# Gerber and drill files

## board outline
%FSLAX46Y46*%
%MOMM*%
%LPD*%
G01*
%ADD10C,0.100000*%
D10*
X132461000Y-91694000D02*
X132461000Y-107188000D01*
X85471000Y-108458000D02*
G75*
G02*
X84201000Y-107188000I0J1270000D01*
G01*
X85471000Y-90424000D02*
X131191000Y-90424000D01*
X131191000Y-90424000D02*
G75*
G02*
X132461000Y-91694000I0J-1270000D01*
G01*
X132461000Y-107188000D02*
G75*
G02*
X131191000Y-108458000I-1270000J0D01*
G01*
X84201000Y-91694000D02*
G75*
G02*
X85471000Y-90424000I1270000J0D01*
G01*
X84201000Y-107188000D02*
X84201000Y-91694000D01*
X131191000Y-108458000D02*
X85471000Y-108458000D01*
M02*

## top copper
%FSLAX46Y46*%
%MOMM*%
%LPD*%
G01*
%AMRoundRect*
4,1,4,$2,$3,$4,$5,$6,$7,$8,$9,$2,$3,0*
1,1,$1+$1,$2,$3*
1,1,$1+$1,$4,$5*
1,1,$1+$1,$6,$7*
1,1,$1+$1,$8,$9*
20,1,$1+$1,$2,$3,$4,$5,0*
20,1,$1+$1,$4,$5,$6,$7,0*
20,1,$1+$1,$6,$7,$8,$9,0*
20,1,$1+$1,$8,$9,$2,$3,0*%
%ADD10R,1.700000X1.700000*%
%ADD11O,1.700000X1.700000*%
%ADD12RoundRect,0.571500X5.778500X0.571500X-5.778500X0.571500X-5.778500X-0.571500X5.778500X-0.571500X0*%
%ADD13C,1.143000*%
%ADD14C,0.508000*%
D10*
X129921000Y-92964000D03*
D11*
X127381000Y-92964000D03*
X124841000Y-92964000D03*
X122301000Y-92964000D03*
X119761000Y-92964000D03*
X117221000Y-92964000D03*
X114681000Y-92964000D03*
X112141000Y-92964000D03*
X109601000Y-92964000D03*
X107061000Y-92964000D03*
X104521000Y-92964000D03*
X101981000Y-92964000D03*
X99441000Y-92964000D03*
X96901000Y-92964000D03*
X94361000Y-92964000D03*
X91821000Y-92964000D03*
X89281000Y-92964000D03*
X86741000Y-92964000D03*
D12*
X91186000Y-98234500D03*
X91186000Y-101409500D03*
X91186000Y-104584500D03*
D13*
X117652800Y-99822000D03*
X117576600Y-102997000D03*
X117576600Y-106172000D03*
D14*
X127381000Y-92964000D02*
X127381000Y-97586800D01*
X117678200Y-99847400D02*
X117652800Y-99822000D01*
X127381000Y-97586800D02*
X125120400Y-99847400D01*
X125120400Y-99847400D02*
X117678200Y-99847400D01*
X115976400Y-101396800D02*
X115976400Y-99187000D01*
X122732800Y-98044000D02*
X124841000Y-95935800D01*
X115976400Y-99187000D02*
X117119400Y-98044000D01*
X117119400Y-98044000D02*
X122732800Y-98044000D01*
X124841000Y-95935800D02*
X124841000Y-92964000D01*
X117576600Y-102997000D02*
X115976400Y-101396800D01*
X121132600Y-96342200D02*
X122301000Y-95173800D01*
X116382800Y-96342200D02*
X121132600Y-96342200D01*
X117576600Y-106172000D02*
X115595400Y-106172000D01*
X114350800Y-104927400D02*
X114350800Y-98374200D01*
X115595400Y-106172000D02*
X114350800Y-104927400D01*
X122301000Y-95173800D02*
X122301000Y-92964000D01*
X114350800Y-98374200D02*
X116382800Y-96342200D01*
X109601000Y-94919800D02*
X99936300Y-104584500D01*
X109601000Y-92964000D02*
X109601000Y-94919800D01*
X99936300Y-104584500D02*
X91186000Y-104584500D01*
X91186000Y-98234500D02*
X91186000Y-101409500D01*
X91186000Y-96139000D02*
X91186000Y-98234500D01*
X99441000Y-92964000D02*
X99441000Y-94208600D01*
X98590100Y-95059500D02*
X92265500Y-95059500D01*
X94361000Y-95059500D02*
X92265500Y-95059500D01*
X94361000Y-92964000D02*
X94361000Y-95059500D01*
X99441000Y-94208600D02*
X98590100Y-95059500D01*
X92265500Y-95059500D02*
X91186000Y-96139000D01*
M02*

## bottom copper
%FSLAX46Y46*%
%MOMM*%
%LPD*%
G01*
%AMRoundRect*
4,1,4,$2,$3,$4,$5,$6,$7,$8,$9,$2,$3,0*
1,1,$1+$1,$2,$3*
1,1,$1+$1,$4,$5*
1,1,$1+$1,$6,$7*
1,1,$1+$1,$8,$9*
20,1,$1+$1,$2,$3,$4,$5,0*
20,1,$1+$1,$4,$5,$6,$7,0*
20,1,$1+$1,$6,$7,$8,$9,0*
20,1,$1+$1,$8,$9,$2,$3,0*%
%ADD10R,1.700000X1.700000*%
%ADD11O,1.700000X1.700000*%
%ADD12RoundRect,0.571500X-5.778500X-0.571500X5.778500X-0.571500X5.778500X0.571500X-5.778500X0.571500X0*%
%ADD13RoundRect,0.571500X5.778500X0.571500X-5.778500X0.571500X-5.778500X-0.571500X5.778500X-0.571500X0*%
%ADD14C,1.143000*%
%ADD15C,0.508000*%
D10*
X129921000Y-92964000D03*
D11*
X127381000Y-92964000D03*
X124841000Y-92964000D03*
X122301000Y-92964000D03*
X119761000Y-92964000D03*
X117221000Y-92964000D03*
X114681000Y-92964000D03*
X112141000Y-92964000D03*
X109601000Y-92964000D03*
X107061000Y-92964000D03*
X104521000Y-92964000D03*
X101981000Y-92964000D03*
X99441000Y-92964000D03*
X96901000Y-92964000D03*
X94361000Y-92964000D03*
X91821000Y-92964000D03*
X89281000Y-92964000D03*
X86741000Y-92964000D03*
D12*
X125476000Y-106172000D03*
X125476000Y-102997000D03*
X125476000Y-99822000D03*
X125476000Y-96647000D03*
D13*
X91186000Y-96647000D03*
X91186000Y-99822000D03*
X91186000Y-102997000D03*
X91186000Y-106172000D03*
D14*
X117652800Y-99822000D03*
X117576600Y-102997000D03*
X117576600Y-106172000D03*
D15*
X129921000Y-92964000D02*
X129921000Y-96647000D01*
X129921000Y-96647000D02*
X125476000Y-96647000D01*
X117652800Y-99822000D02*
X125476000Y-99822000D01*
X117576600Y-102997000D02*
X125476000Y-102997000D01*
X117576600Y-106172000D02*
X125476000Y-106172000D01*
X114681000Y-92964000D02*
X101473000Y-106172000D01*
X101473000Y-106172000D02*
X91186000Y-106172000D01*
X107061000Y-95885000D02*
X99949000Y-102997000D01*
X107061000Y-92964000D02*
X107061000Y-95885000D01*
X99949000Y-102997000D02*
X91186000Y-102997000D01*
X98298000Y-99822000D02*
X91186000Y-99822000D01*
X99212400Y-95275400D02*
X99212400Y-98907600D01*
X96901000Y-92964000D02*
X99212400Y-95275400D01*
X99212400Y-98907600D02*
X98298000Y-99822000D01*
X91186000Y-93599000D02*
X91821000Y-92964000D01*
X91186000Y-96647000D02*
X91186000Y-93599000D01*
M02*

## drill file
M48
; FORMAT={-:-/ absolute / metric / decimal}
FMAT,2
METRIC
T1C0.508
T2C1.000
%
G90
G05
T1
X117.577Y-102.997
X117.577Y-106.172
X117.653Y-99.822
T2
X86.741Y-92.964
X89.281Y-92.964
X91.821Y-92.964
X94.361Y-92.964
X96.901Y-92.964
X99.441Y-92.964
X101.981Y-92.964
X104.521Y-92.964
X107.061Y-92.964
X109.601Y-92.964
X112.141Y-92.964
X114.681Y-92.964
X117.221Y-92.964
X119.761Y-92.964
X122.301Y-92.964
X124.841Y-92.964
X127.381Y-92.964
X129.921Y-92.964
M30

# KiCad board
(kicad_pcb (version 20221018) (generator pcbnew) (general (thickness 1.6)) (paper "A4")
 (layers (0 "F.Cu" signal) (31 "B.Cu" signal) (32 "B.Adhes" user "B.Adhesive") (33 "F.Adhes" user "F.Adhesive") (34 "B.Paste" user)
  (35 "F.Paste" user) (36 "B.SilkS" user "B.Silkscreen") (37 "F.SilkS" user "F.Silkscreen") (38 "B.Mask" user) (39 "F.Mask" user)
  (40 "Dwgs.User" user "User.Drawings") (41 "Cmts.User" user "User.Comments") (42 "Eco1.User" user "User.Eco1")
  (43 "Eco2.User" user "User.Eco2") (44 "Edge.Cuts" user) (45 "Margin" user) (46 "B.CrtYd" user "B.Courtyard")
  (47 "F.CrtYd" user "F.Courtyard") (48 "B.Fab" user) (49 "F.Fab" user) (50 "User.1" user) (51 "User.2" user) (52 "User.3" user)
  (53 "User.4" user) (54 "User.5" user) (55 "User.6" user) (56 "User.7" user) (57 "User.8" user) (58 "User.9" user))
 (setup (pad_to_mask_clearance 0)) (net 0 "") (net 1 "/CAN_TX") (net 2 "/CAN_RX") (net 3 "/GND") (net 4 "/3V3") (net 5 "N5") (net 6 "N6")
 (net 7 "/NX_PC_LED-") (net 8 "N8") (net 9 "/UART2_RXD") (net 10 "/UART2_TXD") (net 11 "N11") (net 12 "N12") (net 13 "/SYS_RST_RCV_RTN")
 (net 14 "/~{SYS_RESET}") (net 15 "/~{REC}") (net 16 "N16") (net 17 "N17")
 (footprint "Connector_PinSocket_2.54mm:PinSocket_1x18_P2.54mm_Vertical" (layer "F.Cu") (at 129.921 92.964 -90)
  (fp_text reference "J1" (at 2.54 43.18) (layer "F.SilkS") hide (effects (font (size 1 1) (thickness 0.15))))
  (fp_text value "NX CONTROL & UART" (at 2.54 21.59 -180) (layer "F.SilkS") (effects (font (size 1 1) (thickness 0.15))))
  (pad "1" thru_hole rect (at 0 0 270) (size 1.7 1.7) (drill 1) (layers "*.Cu" "*.Mask") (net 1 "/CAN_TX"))
  (pad "2" thru_hole oval (at 0 2.54 270) (size 1.7 1.7) (drill 1) (layers "*.Cu" "*.Mask") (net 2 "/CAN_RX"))
  (pad "3" thru_hole oval (at 0 5.08 270) (size 1.7 1.7) (drill 1) (layers "*.Cu" "*.Mask") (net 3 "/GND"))
  (pad "4" thru_hole oval (at 0 7.62 270) (size 1.7 1.7) (drill 1) (layers "*.Cu" "*.Mask") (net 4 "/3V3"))
  (pad "5" thru_hole oval (at 0 10.16 270) (size 1.7 1.7) (drill 1) (layers "*.Cu" "*.Mask") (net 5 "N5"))
  (pad "6" thru_hole oval (at 0 12.7 270) (size 1.7 1.7) (drill 1) (layers "*.Cu" "*.Mask") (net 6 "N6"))
  (pad "7" thru_hole oval (at 0 15.24 270) (size 1.7 1.7) (drill 1) (layers "*.Cu" "*.Mask") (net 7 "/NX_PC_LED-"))
  (pad "8" thru_hole oval (at 0 17.78 270) (size 1.7 1.7) (drill 1) (layers "*.Cu" "*.Mask") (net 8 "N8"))
  (pad "9" thru_hole oval (at 0 20.32 270) (size 1.7 1.7) (drill 1) (layers "*.Cu" "*.Mask") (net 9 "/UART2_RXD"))
  (pad "10" thru_hole oval (at 0 22.86 270) (size 1.7 1.7) (drill 1) (layers "*.Cu" "*.Mask") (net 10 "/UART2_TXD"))
  (pad "11" thru_hole oval (at 0 25.4 270) (size 1.7 1.7) (drill 1) (layers "*.Cu" "*.Mask") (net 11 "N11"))
  (pad "12" thru_hole oval (at 0 27.94 270) (size 1.7 1.7) (drill 1) (layers "*.Cu" "*.Mask") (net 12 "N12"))
  (pad "13" thru_hole oval (at 0 30.48 270) (size 1.7 1.7) (drill 1) (layers "*.Cu" "*.Mask") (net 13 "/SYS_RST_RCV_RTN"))
  (pad "14" thru_hole oval (at 0 33.02 270) (size 1.7 1.7) (drill 1) (layers "*.Cu" "*.Mask") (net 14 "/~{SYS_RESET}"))
  (pad "15" thru_hole oval (at 0 35.56 270) (size 1.7 1.7) (drill 1) (layers "*.Cu" "*.Mask") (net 13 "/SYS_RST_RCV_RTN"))
  (pad "16" thru_hole oval (at 0 38.1 270) (size 1.7 1.7) (drill 1) (layers "*.Cu" "*.Mask") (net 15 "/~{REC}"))
  (pad "17" thru_hole oval (at 0 40.64 270) (size 1.7 1.7) (drill 1) (layers "*.Cu" "*.Mask") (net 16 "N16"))
  (pad "18" thru_hole oval (at 0 43.18 270) (size 1.7 1.7) (drill 1) (layers "*.Cu" "*.Mask") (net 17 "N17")))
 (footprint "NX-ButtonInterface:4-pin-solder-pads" (layer "B.Cu") (at 125.476 106.172)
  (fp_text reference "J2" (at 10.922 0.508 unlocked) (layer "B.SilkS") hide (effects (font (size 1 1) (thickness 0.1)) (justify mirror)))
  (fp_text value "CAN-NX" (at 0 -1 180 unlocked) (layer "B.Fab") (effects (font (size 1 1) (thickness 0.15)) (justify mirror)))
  (pad "1" smd roundrect (at 0 0) (size 12.7 2.286) (layers "B.Cu" "B.Paste" "B.Mask") (roundrect_rratio 0.25) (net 4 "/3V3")
   (thermal_bridge_angle 45))
  (pad "2" smd roundrect (at 0 -3.175) (size 12.7 2.286) (layers "B.Cu" "B.Paste" "B.Mask") (roundrect_rratio 0.25) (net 3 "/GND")
   (thermal_bridge_angle 45))
  (pad "3" smd roundrect (at 0 -6.35) (size 12.7 2.286) (layers "B.Cu" "B.Paste" "B.Mask") (roundrect_rratio 0.25) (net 2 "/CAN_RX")
   (thermal_bridge_angle 45))
  (pad "4" smd roundrect (at 0 -9.525) (size 12.7 2.286) (layers "B.Cu" "B.Paste" "B.Mask") (roundrect_rratio 0.25) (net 1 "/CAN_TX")
   (thermal_bridge_angle 45)))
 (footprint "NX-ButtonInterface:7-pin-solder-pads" (layer "B.Cu") (at 91.186 96.647 180)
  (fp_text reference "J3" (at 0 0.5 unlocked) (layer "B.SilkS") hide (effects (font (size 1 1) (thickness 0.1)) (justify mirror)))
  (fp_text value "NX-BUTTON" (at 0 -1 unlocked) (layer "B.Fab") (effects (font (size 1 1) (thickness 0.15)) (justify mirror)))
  (pad "1" smd roundrect (at 0 0 180) (size 12.7 2.286) (layers "B.Cu" "B.Paste" "B.Mask") (roundrect_rratio 0.25) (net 15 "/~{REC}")
   (thermal_bridge_angle 45))
  (pad "2" smd roundrect (at 0 -1.5875 180) (size 12.7 2.286) (layers "F.Cu" "F.Paste" "F.Mask") (roundrect_rratio 0.25)
   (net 13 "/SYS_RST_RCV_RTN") (thermal_bridge_angle 45))
  (pad "3" smd roundrect (at 0 -3.175 180) (size 12.7 2.286) (layers "B.Cu" "B.Paste" "B.Mask") (roundrect_rratio 0.25)
   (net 14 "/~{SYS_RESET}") (thermal_bridge_angle 45))
  (pad "4" smd roundrect (at 0 -4.7625 180) (size 12.7 2.286) (layers "F.Cu" "F.Paste" "F.Mask") (roundrect_rratio 0.25)
   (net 13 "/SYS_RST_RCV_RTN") (thermal_bridge_angle 45))
  (pad "5" smd roundrect (at 0 -6.35 180) (size 12.7 2.286) (layers "B.Cu" "B.Paste" "B.Mask") (roundrect_rratio 0.25) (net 10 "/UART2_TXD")
   (thermal_bridge_angle 45))
  (pad "6" smd roundrect (at 0 -7.9375 180) (size 12.7 2.286) (layers "F.Cu" "F.Paste" "F.Mask") (roundrect_rratio 0.25)
   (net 9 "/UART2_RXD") (thermal_bridge_angle 45))
  (pad "7" smd roundrect (at 0 -9.525 180) (size 12.7 2.286) (layers "B.Cu" "B.Paste" "B.Mask") (roundrect_rratio 0.25)
   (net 7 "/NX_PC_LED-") (thermal_bridge_angle 45)))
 (gr_line (start 132.461 91.694) (end 132.461 107.188) (stroke (width 0.1) (type default)) (layer "Edge.Cuts"))
 (gr_arc (start 85.471 108.458) (mid 84.572974 108.086026) (end 84.201 107.188) (stroke (width 0.1) (type default)) (layer "Edge.Cuts"))
 (gr_line (start 85.471 90.424) (end 131.191 90.424) (stroke (width 0.1) (type default)) (layer "Edge.Cuts"))
 (gr_arc (start 131.191 90.424) (mid 132.089026 90.795974) (end 132.461 91.694) (stroke (width 0.1) (type default)) (layer "Edge.Cuts"))
 (gr_arc (start 132.461 107.188) (mid 132.089026 108.086026) (end 131.191 108.458) (stroke (width 0.1) (type default)) (layer "Edge.Cuts"))
 (gr_arc (start 84.201 91.694) (mid 84.572974 90.795974) (end 85.471 90.424) (stroke (width 0.1) (type default)) (layer "Edge.Cuts"))
 (gr_line (start 84.201 107.188) (end 84.201 91.694) (stroke (width 0.1) (type default)) (layer "Edge.Cuts"))
 (gr_line (start 131.191 108.458) (end 85.471 108.458) (stroke (width 0.1) (type default)) (layer "Edge.Cuts"))
 (segment (start 129.921 92.964) (end 129.921 96.647) (width 0.508) (layer "B.Cu") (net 1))
 (segment (start 129.921 96.647) (end 125.476 96.647) (width 0.508) (layer "B.Cu") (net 1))
 (segment (start 127.381 92.964) (end 127.381 97.5868) (width 0.508) (layer "F.Cu") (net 2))
 (segment (start 117.6782 99.8474) (end 117.6528 99.822) (width 0.508) (layer "F.Cu") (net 2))
 (segment (start 127.381 97.5868) (end 125.1204 99.8474) (width 0.508) (layer "F.Cu") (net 2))
 (segment (start 125.1204 99.8474) (end 117.6782 99.8474) (width 0.508) (layer "F.Cu") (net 2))
 (via (at 117.6528 99.822) (size 1.143) (drill 0.508) (layers "F.Cu" "B.Cu") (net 2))
 (segment (start 117.6528 99.822) (end 125.476 99.822) (width 0.508) (layer "B.Cu") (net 2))
 (segment (start 115.9764 101.3968) (end 115.9764 99.187) (width 0.508) (layer "F.Cu") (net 3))
 (segment (start 122.7328 98.044) (end 124.841 95.9358) (width 0.508) (layer "F.Cu") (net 3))
 (segment (start 115.9764 99.187) (end 117.1194 98.044) (width 0.508) (layer "F.Cu") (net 3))
 (segment (start 117.1194 98.044) (end 122.7328 98.044) (width 0.508) (layer "F.Cu") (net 3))
 (segment (start 124.841 95.9358) (end 124.841 92.964) (width 0.508) (layer "F.Cu") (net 3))
 (segment (start 117.5766 102.997) (end 115.9764 101.3968) (width 0.508) (layer "F.Cu") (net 3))
 (via (at 117.5766 102.997) (size 1.143) (drill 0.508) (layers "F.Cu" "B.Cu") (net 3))
 (segment (start 117.5766 102.997) (end 125.476 102.997) (width 0.508) (layer "B.Cu") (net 3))
 (segment (start 121.1326 96.3422) (end 122.301 95.1738) (width 0.508) (layer "F.Cu") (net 4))
 (segment (start 116.3828 96.3422) (end 121.1326 96.3422) (width 0.508) (layer "F.Cu") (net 4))
 (segment (start 117.5766 106.172) (end 115.5954 106.172) (width 0.508) (layer "F.Cu") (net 4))
 (segment (start 114.3508 104.9274) (end 114.3508 98.3742) (width 0.508) (layer "F.Cu") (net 4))
 (segment (start 115.5954 106.172) (end 114.3508 104.9274) (width 0.508) (layer "F.Cu") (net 4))
 (segment (start 122.301 95.1738) (end 122.301 92.964) (width 0.508) (layer "F.Cu") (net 4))
 (segment (start 114.3508 98.3742) (end 116.3828 96.3422) (width 0.508) (layer "F.Cu") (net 4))
 (via (at 117.5766 106.172) (size 1.143) (drill 0.508) (layers "F.Cu" "B.Cu") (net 4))
 (segment (start 117.5766 106.172) (end 125.476 106.172) (width 0.508) (layer "B.Cu") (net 4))
 (segment (start 114.681 92.964) (end 101.473 106.172) (width 0.508) (layer "B.Cu") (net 7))
 (segment (start 101.473 106.172) (end 91.186 106.172) (width 0.508) (layer "B.Cu") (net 7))
 (segment (start 109.601 94.9198) (end 99.9363 104.5845) (width 0.508) (layer "F.Cu") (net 9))
 (segment (start 109.601 92.964) (end 109.601 94.9198) (width 0.508) (layer "F.Cu") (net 9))
 (segment (start 99.9363 104.5845) (end 91.186 104.5845) (width 0.508) (layer "F.Cu") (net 9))
 (segment (start 107.061 95.885) (end 99.949 102.997) (width 0.508) (layer "B.Cu") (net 10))
 (segment (start 107.061 92.964) (end 107.061 95.885) (width 0.508) (layer "B.Cu") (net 10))
 (segment (start 99.949 102.997) (end 91.186 102.997) (width 0.508) (layer "B.Cu") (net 10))
 (segment (start 91.186 98.2345) (end 91.186 101.4095) (width 0.508) (layer "F.Cu") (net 13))
 (segment (start 91.186 96.139) (end 91.186 98.2345) (width 0.508) (layer "F.Cu") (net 13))
 (segment (start 99.441 92.964) (end 99.441 94.2086) (width 0.508) (layer "F.Cu") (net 13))
 (segment (start 98.5901 95.0595) (end 92.2655 95.0595) (width 0.508) (layer "F.Cu") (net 13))
 (segment (start 94.361 95.0595) (end 92.2655 95.0595) (width 0.508) (layer "F.Cu") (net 13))
 (segment (start 94.361 92.964) (end 94.361 95.0595) (width 0.508) (layer "F.Cu") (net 13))
 (segment (start 99.441 94.2086) (end 98.5901 95.0595) (width 0.508) (layer "F.Cu") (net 13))
 (segment (start 92.2655 95.0595) (end 91.186 96.139) (width 0.508) (layer "F.Cu") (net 13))
 (segment (start 98.298 99.822) (end 91.186 99.822) (width 0.508) (layer "B.Cu") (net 14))
 (segment (start 99.2124 95.2754) (end 99.2124 98.9076) (width 0.508) (layer "B.Cu") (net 14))
 (segment (start 96.901 92.964) (end 99.2124 95.2754) (width 0.508) (layer "B.Cu") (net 14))
 (segment (start 99.2124 98.9076) (end 98.298 99.822) (width 0.508) (layer "B.Cu") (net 14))
 (segment (start 91.186 93.599) (end 91.821 92.964) (width 0.508) (layer "B.Cu") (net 15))
 (segment (start 91.186 96.647) (end 91.186 93.599) (width 0.508) (layer "B.Cu") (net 15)))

